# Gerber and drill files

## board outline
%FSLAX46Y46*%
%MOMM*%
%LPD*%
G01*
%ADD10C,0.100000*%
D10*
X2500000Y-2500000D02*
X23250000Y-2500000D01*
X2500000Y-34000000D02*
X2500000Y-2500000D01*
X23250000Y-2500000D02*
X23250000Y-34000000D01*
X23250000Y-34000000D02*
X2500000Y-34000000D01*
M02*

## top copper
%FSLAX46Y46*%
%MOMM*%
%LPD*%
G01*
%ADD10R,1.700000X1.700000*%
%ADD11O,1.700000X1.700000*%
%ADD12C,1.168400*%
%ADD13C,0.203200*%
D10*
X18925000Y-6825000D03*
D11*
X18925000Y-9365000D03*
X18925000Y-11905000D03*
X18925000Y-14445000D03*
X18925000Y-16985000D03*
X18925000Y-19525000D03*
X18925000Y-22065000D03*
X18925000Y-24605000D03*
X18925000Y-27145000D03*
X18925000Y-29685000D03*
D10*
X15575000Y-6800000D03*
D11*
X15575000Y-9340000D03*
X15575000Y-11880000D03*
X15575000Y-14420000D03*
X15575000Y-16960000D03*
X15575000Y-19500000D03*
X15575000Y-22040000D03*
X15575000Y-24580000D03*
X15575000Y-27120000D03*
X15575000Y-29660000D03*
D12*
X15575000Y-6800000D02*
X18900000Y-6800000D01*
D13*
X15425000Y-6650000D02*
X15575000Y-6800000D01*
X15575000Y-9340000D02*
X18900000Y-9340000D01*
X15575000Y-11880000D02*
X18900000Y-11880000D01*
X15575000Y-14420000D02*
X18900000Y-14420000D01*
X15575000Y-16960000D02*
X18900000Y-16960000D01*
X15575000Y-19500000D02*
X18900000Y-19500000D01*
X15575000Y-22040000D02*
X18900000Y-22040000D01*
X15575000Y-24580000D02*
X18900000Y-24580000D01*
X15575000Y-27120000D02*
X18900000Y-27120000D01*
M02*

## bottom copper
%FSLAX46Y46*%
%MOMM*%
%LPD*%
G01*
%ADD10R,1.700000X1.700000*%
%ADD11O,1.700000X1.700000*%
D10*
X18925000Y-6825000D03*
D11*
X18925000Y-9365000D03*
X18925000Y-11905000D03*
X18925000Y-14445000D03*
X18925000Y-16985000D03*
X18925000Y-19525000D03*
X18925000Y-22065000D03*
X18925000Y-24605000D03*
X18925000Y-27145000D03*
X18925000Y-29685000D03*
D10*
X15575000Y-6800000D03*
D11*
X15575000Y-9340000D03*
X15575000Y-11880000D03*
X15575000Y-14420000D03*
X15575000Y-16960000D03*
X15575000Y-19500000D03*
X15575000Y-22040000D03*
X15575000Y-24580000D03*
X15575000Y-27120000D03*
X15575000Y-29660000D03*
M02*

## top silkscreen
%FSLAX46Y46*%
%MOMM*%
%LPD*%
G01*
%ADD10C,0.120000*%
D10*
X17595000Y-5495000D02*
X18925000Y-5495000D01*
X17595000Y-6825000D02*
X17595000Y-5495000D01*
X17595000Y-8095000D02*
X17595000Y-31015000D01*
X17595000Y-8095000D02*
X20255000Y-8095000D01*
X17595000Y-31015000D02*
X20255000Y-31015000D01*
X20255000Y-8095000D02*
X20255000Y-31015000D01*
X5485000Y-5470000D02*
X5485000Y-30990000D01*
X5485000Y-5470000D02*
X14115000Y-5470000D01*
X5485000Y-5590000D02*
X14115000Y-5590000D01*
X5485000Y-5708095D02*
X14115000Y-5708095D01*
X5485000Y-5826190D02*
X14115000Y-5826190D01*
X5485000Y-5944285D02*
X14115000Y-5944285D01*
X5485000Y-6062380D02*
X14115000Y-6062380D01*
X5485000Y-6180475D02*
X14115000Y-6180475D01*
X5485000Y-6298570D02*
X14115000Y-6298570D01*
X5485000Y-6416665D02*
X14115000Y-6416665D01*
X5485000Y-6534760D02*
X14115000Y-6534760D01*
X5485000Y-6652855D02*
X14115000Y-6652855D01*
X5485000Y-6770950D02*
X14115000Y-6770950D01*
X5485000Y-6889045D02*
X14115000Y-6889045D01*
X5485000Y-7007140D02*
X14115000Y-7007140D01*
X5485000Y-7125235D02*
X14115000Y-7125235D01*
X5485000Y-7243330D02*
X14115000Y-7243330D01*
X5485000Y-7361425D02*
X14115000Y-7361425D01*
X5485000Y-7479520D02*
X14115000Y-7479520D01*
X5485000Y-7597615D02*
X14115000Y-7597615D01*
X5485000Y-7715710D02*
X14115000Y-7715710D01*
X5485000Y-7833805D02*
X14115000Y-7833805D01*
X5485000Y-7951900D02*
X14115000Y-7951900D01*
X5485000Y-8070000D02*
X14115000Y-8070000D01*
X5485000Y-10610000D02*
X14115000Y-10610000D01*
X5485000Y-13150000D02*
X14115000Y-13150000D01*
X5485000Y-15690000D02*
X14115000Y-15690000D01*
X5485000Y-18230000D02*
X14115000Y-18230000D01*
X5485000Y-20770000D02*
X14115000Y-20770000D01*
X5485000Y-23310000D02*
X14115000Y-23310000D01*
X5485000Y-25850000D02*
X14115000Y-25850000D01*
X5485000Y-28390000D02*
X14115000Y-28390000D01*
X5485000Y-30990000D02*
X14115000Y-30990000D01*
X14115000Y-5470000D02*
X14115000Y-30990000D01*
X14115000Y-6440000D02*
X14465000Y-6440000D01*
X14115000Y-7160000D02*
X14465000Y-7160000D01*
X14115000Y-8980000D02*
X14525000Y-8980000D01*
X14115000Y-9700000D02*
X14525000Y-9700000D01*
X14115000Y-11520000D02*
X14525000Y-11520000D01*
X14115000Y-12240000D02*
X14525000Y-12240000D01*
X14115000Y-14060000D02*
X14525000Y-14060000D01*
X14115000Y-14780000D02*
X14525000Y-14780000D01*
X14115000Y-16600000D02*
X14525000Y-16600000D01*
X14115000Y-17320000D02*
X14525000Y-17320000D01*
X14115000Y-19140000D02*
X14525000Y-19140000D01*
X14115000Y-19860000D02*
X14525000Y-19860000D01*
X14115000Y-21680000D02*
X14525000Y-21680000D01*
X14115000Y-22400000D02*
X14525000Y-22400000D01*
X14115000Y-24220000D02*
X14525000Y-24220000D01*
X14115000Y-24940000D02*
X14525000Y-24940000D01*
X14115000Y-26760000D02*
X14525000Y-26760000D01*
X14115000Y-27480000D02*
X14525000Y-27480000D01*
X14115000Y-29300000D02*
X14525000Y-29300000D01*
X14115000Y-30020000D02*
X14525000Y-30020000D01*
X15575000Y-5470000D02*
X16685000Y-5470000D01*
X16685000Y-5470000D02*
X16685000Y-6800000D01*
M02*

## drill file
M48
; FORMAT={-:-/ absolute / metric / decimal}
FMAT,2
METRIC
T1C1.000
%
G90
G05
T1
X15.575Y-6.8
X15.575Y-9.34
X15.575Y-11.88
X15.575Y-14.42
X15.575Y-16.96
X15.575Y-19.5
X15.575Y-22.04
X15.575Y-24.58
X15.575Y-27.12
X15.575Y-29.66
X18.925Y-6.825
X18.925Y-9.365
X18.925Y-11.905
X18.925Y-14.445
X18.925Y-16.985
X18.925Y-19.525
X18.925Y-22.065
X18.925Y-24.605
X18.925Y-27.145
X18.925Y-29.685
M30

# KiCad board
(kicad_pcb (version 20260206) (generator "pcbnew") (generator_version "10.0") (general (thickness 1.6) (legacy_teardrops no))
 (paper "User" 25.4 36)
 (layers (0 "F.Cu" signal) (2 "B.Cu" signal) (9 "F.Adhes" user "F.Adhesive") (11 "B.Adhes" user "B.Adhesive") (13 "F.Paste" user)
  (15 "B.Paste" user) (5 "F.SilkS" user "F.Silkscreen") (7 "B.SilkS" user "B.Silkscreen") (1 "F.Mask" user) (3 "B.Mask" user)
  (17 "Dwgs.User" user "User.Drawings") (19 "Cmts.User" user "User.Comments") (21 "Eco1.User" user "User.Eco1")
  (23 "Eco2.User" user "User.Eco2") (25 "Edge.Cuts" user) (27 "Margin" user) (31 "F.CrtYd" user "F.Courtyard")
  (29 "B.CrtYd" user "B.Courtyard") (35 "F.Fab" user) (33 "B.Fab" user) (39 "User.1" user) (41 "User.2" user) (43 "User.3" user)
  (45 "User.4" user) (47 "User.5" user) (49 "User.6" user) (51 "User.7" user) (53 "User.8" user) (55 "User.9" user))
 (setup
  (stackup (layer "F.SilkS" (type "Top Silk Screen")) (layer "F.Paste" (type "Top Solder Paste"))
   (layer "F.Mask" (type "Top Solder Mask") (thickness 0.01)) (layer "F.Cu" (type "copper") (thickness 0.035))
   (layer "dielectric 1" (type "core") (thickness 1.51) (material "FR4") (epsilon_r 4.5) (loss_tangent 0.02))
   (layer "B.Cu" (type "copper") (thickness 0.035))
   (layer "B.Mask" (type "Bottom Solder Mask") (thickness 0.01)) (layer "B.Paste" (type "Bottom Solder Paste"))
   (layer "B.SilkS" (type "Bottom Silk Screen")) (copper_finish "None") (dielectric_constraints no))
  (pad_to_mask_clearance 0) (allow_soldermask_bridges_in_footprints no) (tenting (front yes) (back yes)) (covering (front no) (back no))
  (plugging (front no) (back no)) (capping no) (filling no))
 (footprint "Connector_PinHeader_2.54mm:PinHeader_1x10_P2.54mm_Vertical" (layer "F.Cu") (at 18.925 6.825)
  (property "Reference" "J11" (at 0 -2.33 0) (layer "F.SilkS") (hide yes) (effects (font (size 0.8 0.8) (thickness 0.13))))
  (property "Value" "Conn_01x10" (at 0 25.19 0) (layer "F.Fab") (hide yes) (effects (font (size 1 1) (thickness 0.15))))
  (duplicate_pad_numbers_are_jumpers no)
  (fp_line (start -1.33 -1.33) (end 0 -1.33) (stroke (width 0.12) (type solid)) (layer "F.SilkS"))
  (fp_line (start -1.33 0) (end -1.33 -1.33) (stroke (width 0.12) (type solid)) (layer "F.SilkS"))
  (fp_line (start -1.33 1.27) (end -1.33 24.19) (stroke (width 0.12) (type solid)) (layer "F.SilkS"))
  (fp_line (start -1.33 1.27) (end 1.33 1.27) (stroke (width 0.12) (type solid)) (layer "F.SilkS"))
  (fp_line (start -1.33 24.19) (end 1.33 24.19) (stroke (width 0.12) (type solid)) (layer "F.SilkS"))
  (fp_line (start 1.33 1.27) (end 1.33 24.19) (stroke (width 0.12) (type solid)) (layer "F.SilkS"))
  (pad "1" thru_hole rect (at 0 0) (size 1.7 1.7) (drill 1) (layers "*.Cu" "*.Mask") (remove_unused_layers no) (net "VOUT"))
  (pad "2" thru_hole oval (at 0 2.54) (size 1.7 1.7) (drill 1) (layers "*.Cu" "*.Mask") (remove_unused_layers no) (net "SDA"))
  (pad "3" thru_hole oval (at 0 5.08) (size 1.7 1.7) (drill 1) (layers "*.Cu" "*.Mask") (remove_unused_layers no) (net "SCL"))
  (pad "4" thru_hole oval (at 0 7.62) (size 1.7 1.7) (drill 1) (layers "*.Cu" "*.Mask") (remove_unused_layers no) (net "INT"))
  (pad "5" thru_hole oval (at 0 10.16) (size 1.7 1.7) (drill 1) (layers "*.Cu" "*.Mask") (remove_unused_layers no) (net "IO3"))
  (pad "6" thru_hole oval (at 0 12.7) (size 1.7 1.7) (drill 1) (layers "*.Cu" "*.Mask") (remove_unused_layers no) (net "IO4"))
  (pad "7" thru_hole oval (at 0 15.24) (size 1.7 1.7) (drill 1) (layers "*.Cu" "*.Mask") (remove_unused_layers no) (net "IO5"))
  (pad "8" thru_hole oval (at 0 17.78) (size 1.7 1.7) (drill 1) (layers "*.Cu" "*.Mask") (remove_unused_layers no) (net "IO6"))
  (pad "9" thru_hole oval (at 0 20.32) (size 1.7 1.7) (drill 1) (layers "*.Cu" "*.Mask") (remove_unused_layers no) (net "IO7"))
  (pad "10" thru_hole oval (at 0 22.86) (size 1.7 1.7) (drill 1) (layers "*.Cu" "*.Mask") (remove_unused_layers no) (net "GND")))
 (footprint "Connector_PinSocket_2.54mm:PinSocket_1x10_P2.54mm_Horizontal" (layer "F.Cu") (at 15.575 6.8)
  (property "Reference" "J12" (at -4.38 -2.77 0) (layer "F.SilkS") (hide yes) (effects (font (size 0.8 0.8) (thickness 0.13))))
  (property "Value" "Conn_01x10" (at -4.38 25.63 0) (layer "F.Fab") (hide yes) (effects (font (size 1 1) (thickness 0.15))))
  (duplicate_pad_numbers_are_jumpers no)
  (fp_line (start -10.09 -1.33) (end -10.09 24.19) (stroke (width 0.12) (type solid)) (layer "F.SilkS"))
  (fp_line (start -10.09 -1.33) (end -1.46 -1.33) (stroke (width 0.12) (type solid)) (layer "F.SilkS"))
  (fp_line (start -10.09 -1.21) (end -1.46 -1.21) (stroke (width 0.12) (type solid)) (layer "F.SilkS"))
  (fp_line (start -10.09 -1.091905) (end -1.46 -1.091905) (stroke (width 0.12) (type solid)) (layer "F.SilkS"))
  (fp_line (start -10.09 -0.97381) (end -1.46 -0.97381) (stroke (width 0.12) (type solid)) (layer "F.SilkS"))
  (fp_line (start -10.09 -0.855715) (end -1.46 -0.855715) (stroke (width 0.12) (type solid)) (layer "F.SilkS"))
  (fp_line (start -10.09 -0.73762) (end -1.46 -0.73762) (stroke (width 0.12) (type solid)) (layer "F.SilkS"))
  (fp_line (start -10.09 -0.619525) (end -1.46 -0.619525) (stroke (width 0.12) (type solid)) (layer "F.SilkS"))
  (fp_line (start -10.09 -0.50143) (end -1.46 -0.50143) (stroke (width 0.12) (type solid)) (layer "F.SilkS"))
  (fp_line (start -10.09 -0.383335) (end -1.46 -0.383335) (stroke (width 0.12) (type solid)) (layer "F.SilkS"))
  (fp_line (start -10.09 -0.26524) (end -1.46 -0.26524) (stroke (width 0.12) (type solid)) (layer "F.SilkS"))
  (fp_line (start -10.09 -0.147145) (end -1.46 -0.147145) (stroke (width 0.12) (type solid)) (layer "F.SilkS"))
  (fp_line (start -10.09 -0.02905) (end -1.46 -0.02905) (stroke (width 0.12) (type solid)) (layer "F.SilkS"))
  (fp_line (start -10.09 0.089045) (end -1.46 0.089045) (stroke (width 0.12) (type solid)) (layer "F.SilkS"))
  (fp_line (start -10.09 0.20714) (end -1.46 0.20714) (stroke (width 0.12) (type solid)) (layer "F.SilkS"))
  (fp_line (start -10.09 0.325235) (end -1.46 0.325235) (stroke (width 0.12) (type solid)) (layer "F.SilkS"))
  (fp_line (start -10.09 0.44333) (end -1.46 0.44333) (stroke (width 0.12) (type solid)) (layer "F.SilkS"))
  (fp_line (start -10.09 0.561425) (end -1.46 0.561425) (stroke (width 0.12) (type solid)) (layer "F.SilkS"))
  (fp_line (start -10.09 0.67952) (end -1.46 0.67952) (stroke (width 0.12) (type solid)) (layer "F.SilkS"))
  (fp_line (start -10.09 0.797615) (end -1.46 0.797615) (stroke (width 0.12) (type solid)) (layer "F.SilkS"))
  (fp_line (start -10.09 0.91571) (end -1.46 0.91571) (stroke (width 0.12) (type solid)) (layer "F.SilkS"))
  (fp_line (start -10.09 1.033805) (end -1.46 1.033805) (stroke (width 0.12) (type solid)) (layer "F.SilkS"))
  (fp_line (start -10.09 1.1519) (end -1.46 1.1519) (stroke (width 0.12) (type solid)) (layer "F.SilkS"))
  (fp_line (start -10.09 1.27) (end -1.46 1.27) (stroke (width 0.12) (type solid)) (layer "F.SilkS"))
  (fp_line (start -10.09 3.81) (end -1.46 3.81) (stroke (width 0.12) (type solid)) (layer "F.SilkS"))
  (fp_line (start -10.09 6.35) (end -1.46 6.35) (stroke (width 0.12) (type solid)) (layer "F.SilkS"))
  (fp_line (start -10.09 8.89) (end -1.46 8.89) (stroke (width 0.12) (type solid)) (layer "F.SilkS"))
  (fp_line (start -10.09 11.43) (end -1.46 11.43) (stroke (width 0.12) (type solid)) (layer "F.SilkS"))
  (fp_line (start -10.09 13.97) (end -1.46 13.97) (stroke (width 0.12) (type solid)) (layer "F.SilkS"))
  (fp_line (start -10.09 16.51) (end -1.46 16.51) (stroke (width 0.12) (type solid)) (layer "F.SilkS"))
  (fp_line (start -10.09 19.05) (end -1.46 19.05) (stroke (width 0.12) (type solid)) (layer "F.SilkS"))
  (fp_line (start -10.09 21.59) (end -1.46 21.59) (stroke (width 0.12) (type solid)) (layer "F.SilkS"))
  (fp_line (start -10.09 24.19) (end -1.46 24.19) (stroke (width 0.12) (type solid)) (layer "F.SilkS"))
  (fp_line (start -1.46 -1.33) (end -1.46 24.19) (stroke (width 0.12) (type solid)) (layer "F.SilkS"))
  (fp_line (start -1.46 -0.36) (end -1.11 -0.36) (stroke (width 0.12) (type solid)) (layer "F.SilkS"))
  (fp_line (start -1.46 0.36) (end -1.11 0.36) (stroke (width 0.12) (type solid)) (layer "F.SilkS"))
  (fp_line (start -1.46 2.18) (end -1.05 2.18) (stroke (width 0.12) (type solid)) (layer "F.SilkS"))
  (fp_line (start -1.46 2.9) (end -1.05 2.9) (stroke (width 0.12) (type solid)) (layer "F.SilkS"))
  (fp_line (start -1.46 4.72) (end -1.05 4.72) (stroke (width 0.12) (type solid)) (layer "F.SilkS"))
  (fp_line (start -1.46 5.44) (end -1.05 5.44) (stroke (width 0.12) (type solid)) (layer "F.SilkS"))
  (fp_line (start -1.46 7.26) (end -1.05 7.26) (stroke (width 0.12) (type solid)) (layer "F.SilkS"))
  (fp_line (start -1.46 7.98) (end -1.05 7.98) (stroke (width 0.12) (type solid)) (layer "F.SilkS"))
  (fp_line (start -1.46 9.8) (end -1.05 9.8) (stroke (width 0.12) (type solid)) (layer "F.SilkS"))
  (fp_line (start -1.46 10.52) (end -1.05 10.52) (stroke (width 0.12) (type solid)) (layer "F.SilkS"))
  (fp_line (start -1.46 12.34) (end -1.05 12.34) (stroke (width 0.12) (type solid)) (layer "F.SilkS"))
  (fp_line (start -1.46 13.06) (end -1.05 13.06) (stroke (width 0.12) (type solid)) (layer "F.SilkS"))
  (fp_line (start -1.46 14.88) (end -1.05 14.88) (stroke (width 0.12) (type solid)) (layer "F.SilkS"))
  (fp_line (start -1.46 15.6) (end -1.05 15.6) (stroke (width 0.12) (type solid)) (layer "F.SilkS"))
  (fp_line (start -1.46 17.42) (end -1.05 17.42) (stroke (width 0.12) (type solid)) (layer "F.SilkS"))
  (fp_line (start -1.46 18.14) (end -1.05 18.14) (stroke (width 0.12) (type solid)) (layer "F.SilkS"))
  (fp_line (start -1.46 19.96) (end -1.05 19.96) (stroke (width 0.12) (type solid)) (layer "F.SilkS"))
  (fp_line (start -1.46 20.68) (end -1.05 20.68) (stroke (width 0.12) (type solid)) (layer "F.SilkS"))
  (fp_line (start -1.46 22.5) (end -1.05 22.5) (stroke (width 0.12) (type solid)) (layer "F.SilkS"))
  (fp_line (start -1.46 23.22) (end -1.05 23.22) (stroke (width 0.12) (type solid)) (layer "F.SilkS"))
  (fp_line (start 0 -1.33) (end 1.11 -1.33) (stroke (width 0.12) (type solid)) (layer "F.SilkS"))
  (fp_line (start 1.11 -1.33) (end 1.11 0) (stroke (width 0.12) (type solid)) (layer "F.SilkS"))
  (pad "1" thru_hole rect (at 0 0) (size 1.7 1.7) (drill 1) (layers "*.Cu" "*.Mask") (remove_unused_layers no) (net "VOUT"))
  (pad "2" thru_hole oval (at 0 2.54) (size 1.7 1.7) (drill 1) (layers "*.Cu" "*.Mask") (remove_unused_layers no) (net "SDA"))
  (pad "3" thru_hole oval (at 0 5.08) (size 1.7 1.7) (drill 1) (layers "*.Cu" "*.Mask") (remove_unused_layers no) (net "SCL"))
  (pad "4" thru_hole oval (at 0 7.62) (size 1.7 1.7) (drill 1) (layers "*.Cu" "*.Mask") (remove_unused_layers no) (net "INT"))
  (pad "5" thru_hole oval (at 0 10.16) (size 1.7 1.7) (drill 1) (layers "*.Cu" "*.Mask") (remove_unused_layers no) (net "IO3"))
  (pad "6" thru_hole oval (at 0 12.7) (size 1.7 1.7) (drill 1) (layers "*.Cu" "*.Mask") (remove_unused_layers no) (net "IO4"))
  (pad "7" thru_hole oval (at 0 15.24) (size 1.7 1.7) (drill 1) (layers "*.Cu" "*.Mask") (remove_unused_layers no) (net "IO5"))
  (pad "8" thru_hole oval (at 0 17.78) (size 1.7 1.7) (drill 1) (layers "*.Cu" "*.Mask") (remove_unused_layers no) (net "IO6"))
  (pad "9" thru_hole oval (at 0 20.32) (size 1.7 1.7) (drill 1) (layers "*.Cu" "*.Mask") (remove_unused_layers no) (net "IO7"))
  (pad "10" thru_hole oval (at 0 22.86) (size 1.7 1.7) (drill 1) (layers "*.Cu" "*.Mask") (remove_unused_layers no) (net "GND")))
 (gr_line (start 2.5 2.5) (end 23.25 2.5) (stroke (width 0.1) (type default)) (layer "Edge.Cuts"))
 (gr_line (start 2.5 34) (end 2.5 2.5) (stroke (width 0.1) (type default)) (layer "Edge.Cuts"))
 (gr_line (start 23.25 2.5) (end 23.25 34) (stroke (width 0.1) (type default)) (layer "Edge.Cuts"))
 (gr_line (start 23.25 34) (end 2.5 34) (stroke (width 0.1) (type default)) (layer "Edge.Cuts"))
 (segment (start 15.575 6.8) (end 18.9 6.8) (width 1.1684) (layer "F.Cu") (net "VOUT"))
 (segment (start 15.425 6.65) (end 15.575 6.8) (width 0.2032) (layer "F.Cu") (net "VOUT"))
 (segment (start 15.575 9.34) (end 18.9 9.34) (width 0.2032) (layer "F.Cu") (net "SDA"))
 (segment (start 15.575 11.88) (end 18.9 11.88) (width 0.2032) (layer "F.Cu") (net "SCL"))
 (segment (start 15.575 14.42) (end 18.9 14.42) (width 0.2032) (layer "F.Cu") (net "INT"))
 (segment (start 15.575 16.96) (end 18.9 16.96) (width 0.2032) (layer "F.Cu") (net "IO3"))
 (segment (start 15.575 19.5) (end 18.9 19.5) (width 0.2032) (layer "F.Cu") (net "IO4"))
 (segment (start 15.575 22.04) (end 18.9 22.04) (width 0.2032) (layer "F.Cu") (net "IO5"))
 (segment (start 15.575 24.58) (end 18.9 24.58) (width 0.2032) (layer "F.Cu") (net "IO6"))
 (segment (start 15.575 27.12) (end 18.9 27.12) (width 0.2032) (layer "F.Cu") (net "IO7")))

